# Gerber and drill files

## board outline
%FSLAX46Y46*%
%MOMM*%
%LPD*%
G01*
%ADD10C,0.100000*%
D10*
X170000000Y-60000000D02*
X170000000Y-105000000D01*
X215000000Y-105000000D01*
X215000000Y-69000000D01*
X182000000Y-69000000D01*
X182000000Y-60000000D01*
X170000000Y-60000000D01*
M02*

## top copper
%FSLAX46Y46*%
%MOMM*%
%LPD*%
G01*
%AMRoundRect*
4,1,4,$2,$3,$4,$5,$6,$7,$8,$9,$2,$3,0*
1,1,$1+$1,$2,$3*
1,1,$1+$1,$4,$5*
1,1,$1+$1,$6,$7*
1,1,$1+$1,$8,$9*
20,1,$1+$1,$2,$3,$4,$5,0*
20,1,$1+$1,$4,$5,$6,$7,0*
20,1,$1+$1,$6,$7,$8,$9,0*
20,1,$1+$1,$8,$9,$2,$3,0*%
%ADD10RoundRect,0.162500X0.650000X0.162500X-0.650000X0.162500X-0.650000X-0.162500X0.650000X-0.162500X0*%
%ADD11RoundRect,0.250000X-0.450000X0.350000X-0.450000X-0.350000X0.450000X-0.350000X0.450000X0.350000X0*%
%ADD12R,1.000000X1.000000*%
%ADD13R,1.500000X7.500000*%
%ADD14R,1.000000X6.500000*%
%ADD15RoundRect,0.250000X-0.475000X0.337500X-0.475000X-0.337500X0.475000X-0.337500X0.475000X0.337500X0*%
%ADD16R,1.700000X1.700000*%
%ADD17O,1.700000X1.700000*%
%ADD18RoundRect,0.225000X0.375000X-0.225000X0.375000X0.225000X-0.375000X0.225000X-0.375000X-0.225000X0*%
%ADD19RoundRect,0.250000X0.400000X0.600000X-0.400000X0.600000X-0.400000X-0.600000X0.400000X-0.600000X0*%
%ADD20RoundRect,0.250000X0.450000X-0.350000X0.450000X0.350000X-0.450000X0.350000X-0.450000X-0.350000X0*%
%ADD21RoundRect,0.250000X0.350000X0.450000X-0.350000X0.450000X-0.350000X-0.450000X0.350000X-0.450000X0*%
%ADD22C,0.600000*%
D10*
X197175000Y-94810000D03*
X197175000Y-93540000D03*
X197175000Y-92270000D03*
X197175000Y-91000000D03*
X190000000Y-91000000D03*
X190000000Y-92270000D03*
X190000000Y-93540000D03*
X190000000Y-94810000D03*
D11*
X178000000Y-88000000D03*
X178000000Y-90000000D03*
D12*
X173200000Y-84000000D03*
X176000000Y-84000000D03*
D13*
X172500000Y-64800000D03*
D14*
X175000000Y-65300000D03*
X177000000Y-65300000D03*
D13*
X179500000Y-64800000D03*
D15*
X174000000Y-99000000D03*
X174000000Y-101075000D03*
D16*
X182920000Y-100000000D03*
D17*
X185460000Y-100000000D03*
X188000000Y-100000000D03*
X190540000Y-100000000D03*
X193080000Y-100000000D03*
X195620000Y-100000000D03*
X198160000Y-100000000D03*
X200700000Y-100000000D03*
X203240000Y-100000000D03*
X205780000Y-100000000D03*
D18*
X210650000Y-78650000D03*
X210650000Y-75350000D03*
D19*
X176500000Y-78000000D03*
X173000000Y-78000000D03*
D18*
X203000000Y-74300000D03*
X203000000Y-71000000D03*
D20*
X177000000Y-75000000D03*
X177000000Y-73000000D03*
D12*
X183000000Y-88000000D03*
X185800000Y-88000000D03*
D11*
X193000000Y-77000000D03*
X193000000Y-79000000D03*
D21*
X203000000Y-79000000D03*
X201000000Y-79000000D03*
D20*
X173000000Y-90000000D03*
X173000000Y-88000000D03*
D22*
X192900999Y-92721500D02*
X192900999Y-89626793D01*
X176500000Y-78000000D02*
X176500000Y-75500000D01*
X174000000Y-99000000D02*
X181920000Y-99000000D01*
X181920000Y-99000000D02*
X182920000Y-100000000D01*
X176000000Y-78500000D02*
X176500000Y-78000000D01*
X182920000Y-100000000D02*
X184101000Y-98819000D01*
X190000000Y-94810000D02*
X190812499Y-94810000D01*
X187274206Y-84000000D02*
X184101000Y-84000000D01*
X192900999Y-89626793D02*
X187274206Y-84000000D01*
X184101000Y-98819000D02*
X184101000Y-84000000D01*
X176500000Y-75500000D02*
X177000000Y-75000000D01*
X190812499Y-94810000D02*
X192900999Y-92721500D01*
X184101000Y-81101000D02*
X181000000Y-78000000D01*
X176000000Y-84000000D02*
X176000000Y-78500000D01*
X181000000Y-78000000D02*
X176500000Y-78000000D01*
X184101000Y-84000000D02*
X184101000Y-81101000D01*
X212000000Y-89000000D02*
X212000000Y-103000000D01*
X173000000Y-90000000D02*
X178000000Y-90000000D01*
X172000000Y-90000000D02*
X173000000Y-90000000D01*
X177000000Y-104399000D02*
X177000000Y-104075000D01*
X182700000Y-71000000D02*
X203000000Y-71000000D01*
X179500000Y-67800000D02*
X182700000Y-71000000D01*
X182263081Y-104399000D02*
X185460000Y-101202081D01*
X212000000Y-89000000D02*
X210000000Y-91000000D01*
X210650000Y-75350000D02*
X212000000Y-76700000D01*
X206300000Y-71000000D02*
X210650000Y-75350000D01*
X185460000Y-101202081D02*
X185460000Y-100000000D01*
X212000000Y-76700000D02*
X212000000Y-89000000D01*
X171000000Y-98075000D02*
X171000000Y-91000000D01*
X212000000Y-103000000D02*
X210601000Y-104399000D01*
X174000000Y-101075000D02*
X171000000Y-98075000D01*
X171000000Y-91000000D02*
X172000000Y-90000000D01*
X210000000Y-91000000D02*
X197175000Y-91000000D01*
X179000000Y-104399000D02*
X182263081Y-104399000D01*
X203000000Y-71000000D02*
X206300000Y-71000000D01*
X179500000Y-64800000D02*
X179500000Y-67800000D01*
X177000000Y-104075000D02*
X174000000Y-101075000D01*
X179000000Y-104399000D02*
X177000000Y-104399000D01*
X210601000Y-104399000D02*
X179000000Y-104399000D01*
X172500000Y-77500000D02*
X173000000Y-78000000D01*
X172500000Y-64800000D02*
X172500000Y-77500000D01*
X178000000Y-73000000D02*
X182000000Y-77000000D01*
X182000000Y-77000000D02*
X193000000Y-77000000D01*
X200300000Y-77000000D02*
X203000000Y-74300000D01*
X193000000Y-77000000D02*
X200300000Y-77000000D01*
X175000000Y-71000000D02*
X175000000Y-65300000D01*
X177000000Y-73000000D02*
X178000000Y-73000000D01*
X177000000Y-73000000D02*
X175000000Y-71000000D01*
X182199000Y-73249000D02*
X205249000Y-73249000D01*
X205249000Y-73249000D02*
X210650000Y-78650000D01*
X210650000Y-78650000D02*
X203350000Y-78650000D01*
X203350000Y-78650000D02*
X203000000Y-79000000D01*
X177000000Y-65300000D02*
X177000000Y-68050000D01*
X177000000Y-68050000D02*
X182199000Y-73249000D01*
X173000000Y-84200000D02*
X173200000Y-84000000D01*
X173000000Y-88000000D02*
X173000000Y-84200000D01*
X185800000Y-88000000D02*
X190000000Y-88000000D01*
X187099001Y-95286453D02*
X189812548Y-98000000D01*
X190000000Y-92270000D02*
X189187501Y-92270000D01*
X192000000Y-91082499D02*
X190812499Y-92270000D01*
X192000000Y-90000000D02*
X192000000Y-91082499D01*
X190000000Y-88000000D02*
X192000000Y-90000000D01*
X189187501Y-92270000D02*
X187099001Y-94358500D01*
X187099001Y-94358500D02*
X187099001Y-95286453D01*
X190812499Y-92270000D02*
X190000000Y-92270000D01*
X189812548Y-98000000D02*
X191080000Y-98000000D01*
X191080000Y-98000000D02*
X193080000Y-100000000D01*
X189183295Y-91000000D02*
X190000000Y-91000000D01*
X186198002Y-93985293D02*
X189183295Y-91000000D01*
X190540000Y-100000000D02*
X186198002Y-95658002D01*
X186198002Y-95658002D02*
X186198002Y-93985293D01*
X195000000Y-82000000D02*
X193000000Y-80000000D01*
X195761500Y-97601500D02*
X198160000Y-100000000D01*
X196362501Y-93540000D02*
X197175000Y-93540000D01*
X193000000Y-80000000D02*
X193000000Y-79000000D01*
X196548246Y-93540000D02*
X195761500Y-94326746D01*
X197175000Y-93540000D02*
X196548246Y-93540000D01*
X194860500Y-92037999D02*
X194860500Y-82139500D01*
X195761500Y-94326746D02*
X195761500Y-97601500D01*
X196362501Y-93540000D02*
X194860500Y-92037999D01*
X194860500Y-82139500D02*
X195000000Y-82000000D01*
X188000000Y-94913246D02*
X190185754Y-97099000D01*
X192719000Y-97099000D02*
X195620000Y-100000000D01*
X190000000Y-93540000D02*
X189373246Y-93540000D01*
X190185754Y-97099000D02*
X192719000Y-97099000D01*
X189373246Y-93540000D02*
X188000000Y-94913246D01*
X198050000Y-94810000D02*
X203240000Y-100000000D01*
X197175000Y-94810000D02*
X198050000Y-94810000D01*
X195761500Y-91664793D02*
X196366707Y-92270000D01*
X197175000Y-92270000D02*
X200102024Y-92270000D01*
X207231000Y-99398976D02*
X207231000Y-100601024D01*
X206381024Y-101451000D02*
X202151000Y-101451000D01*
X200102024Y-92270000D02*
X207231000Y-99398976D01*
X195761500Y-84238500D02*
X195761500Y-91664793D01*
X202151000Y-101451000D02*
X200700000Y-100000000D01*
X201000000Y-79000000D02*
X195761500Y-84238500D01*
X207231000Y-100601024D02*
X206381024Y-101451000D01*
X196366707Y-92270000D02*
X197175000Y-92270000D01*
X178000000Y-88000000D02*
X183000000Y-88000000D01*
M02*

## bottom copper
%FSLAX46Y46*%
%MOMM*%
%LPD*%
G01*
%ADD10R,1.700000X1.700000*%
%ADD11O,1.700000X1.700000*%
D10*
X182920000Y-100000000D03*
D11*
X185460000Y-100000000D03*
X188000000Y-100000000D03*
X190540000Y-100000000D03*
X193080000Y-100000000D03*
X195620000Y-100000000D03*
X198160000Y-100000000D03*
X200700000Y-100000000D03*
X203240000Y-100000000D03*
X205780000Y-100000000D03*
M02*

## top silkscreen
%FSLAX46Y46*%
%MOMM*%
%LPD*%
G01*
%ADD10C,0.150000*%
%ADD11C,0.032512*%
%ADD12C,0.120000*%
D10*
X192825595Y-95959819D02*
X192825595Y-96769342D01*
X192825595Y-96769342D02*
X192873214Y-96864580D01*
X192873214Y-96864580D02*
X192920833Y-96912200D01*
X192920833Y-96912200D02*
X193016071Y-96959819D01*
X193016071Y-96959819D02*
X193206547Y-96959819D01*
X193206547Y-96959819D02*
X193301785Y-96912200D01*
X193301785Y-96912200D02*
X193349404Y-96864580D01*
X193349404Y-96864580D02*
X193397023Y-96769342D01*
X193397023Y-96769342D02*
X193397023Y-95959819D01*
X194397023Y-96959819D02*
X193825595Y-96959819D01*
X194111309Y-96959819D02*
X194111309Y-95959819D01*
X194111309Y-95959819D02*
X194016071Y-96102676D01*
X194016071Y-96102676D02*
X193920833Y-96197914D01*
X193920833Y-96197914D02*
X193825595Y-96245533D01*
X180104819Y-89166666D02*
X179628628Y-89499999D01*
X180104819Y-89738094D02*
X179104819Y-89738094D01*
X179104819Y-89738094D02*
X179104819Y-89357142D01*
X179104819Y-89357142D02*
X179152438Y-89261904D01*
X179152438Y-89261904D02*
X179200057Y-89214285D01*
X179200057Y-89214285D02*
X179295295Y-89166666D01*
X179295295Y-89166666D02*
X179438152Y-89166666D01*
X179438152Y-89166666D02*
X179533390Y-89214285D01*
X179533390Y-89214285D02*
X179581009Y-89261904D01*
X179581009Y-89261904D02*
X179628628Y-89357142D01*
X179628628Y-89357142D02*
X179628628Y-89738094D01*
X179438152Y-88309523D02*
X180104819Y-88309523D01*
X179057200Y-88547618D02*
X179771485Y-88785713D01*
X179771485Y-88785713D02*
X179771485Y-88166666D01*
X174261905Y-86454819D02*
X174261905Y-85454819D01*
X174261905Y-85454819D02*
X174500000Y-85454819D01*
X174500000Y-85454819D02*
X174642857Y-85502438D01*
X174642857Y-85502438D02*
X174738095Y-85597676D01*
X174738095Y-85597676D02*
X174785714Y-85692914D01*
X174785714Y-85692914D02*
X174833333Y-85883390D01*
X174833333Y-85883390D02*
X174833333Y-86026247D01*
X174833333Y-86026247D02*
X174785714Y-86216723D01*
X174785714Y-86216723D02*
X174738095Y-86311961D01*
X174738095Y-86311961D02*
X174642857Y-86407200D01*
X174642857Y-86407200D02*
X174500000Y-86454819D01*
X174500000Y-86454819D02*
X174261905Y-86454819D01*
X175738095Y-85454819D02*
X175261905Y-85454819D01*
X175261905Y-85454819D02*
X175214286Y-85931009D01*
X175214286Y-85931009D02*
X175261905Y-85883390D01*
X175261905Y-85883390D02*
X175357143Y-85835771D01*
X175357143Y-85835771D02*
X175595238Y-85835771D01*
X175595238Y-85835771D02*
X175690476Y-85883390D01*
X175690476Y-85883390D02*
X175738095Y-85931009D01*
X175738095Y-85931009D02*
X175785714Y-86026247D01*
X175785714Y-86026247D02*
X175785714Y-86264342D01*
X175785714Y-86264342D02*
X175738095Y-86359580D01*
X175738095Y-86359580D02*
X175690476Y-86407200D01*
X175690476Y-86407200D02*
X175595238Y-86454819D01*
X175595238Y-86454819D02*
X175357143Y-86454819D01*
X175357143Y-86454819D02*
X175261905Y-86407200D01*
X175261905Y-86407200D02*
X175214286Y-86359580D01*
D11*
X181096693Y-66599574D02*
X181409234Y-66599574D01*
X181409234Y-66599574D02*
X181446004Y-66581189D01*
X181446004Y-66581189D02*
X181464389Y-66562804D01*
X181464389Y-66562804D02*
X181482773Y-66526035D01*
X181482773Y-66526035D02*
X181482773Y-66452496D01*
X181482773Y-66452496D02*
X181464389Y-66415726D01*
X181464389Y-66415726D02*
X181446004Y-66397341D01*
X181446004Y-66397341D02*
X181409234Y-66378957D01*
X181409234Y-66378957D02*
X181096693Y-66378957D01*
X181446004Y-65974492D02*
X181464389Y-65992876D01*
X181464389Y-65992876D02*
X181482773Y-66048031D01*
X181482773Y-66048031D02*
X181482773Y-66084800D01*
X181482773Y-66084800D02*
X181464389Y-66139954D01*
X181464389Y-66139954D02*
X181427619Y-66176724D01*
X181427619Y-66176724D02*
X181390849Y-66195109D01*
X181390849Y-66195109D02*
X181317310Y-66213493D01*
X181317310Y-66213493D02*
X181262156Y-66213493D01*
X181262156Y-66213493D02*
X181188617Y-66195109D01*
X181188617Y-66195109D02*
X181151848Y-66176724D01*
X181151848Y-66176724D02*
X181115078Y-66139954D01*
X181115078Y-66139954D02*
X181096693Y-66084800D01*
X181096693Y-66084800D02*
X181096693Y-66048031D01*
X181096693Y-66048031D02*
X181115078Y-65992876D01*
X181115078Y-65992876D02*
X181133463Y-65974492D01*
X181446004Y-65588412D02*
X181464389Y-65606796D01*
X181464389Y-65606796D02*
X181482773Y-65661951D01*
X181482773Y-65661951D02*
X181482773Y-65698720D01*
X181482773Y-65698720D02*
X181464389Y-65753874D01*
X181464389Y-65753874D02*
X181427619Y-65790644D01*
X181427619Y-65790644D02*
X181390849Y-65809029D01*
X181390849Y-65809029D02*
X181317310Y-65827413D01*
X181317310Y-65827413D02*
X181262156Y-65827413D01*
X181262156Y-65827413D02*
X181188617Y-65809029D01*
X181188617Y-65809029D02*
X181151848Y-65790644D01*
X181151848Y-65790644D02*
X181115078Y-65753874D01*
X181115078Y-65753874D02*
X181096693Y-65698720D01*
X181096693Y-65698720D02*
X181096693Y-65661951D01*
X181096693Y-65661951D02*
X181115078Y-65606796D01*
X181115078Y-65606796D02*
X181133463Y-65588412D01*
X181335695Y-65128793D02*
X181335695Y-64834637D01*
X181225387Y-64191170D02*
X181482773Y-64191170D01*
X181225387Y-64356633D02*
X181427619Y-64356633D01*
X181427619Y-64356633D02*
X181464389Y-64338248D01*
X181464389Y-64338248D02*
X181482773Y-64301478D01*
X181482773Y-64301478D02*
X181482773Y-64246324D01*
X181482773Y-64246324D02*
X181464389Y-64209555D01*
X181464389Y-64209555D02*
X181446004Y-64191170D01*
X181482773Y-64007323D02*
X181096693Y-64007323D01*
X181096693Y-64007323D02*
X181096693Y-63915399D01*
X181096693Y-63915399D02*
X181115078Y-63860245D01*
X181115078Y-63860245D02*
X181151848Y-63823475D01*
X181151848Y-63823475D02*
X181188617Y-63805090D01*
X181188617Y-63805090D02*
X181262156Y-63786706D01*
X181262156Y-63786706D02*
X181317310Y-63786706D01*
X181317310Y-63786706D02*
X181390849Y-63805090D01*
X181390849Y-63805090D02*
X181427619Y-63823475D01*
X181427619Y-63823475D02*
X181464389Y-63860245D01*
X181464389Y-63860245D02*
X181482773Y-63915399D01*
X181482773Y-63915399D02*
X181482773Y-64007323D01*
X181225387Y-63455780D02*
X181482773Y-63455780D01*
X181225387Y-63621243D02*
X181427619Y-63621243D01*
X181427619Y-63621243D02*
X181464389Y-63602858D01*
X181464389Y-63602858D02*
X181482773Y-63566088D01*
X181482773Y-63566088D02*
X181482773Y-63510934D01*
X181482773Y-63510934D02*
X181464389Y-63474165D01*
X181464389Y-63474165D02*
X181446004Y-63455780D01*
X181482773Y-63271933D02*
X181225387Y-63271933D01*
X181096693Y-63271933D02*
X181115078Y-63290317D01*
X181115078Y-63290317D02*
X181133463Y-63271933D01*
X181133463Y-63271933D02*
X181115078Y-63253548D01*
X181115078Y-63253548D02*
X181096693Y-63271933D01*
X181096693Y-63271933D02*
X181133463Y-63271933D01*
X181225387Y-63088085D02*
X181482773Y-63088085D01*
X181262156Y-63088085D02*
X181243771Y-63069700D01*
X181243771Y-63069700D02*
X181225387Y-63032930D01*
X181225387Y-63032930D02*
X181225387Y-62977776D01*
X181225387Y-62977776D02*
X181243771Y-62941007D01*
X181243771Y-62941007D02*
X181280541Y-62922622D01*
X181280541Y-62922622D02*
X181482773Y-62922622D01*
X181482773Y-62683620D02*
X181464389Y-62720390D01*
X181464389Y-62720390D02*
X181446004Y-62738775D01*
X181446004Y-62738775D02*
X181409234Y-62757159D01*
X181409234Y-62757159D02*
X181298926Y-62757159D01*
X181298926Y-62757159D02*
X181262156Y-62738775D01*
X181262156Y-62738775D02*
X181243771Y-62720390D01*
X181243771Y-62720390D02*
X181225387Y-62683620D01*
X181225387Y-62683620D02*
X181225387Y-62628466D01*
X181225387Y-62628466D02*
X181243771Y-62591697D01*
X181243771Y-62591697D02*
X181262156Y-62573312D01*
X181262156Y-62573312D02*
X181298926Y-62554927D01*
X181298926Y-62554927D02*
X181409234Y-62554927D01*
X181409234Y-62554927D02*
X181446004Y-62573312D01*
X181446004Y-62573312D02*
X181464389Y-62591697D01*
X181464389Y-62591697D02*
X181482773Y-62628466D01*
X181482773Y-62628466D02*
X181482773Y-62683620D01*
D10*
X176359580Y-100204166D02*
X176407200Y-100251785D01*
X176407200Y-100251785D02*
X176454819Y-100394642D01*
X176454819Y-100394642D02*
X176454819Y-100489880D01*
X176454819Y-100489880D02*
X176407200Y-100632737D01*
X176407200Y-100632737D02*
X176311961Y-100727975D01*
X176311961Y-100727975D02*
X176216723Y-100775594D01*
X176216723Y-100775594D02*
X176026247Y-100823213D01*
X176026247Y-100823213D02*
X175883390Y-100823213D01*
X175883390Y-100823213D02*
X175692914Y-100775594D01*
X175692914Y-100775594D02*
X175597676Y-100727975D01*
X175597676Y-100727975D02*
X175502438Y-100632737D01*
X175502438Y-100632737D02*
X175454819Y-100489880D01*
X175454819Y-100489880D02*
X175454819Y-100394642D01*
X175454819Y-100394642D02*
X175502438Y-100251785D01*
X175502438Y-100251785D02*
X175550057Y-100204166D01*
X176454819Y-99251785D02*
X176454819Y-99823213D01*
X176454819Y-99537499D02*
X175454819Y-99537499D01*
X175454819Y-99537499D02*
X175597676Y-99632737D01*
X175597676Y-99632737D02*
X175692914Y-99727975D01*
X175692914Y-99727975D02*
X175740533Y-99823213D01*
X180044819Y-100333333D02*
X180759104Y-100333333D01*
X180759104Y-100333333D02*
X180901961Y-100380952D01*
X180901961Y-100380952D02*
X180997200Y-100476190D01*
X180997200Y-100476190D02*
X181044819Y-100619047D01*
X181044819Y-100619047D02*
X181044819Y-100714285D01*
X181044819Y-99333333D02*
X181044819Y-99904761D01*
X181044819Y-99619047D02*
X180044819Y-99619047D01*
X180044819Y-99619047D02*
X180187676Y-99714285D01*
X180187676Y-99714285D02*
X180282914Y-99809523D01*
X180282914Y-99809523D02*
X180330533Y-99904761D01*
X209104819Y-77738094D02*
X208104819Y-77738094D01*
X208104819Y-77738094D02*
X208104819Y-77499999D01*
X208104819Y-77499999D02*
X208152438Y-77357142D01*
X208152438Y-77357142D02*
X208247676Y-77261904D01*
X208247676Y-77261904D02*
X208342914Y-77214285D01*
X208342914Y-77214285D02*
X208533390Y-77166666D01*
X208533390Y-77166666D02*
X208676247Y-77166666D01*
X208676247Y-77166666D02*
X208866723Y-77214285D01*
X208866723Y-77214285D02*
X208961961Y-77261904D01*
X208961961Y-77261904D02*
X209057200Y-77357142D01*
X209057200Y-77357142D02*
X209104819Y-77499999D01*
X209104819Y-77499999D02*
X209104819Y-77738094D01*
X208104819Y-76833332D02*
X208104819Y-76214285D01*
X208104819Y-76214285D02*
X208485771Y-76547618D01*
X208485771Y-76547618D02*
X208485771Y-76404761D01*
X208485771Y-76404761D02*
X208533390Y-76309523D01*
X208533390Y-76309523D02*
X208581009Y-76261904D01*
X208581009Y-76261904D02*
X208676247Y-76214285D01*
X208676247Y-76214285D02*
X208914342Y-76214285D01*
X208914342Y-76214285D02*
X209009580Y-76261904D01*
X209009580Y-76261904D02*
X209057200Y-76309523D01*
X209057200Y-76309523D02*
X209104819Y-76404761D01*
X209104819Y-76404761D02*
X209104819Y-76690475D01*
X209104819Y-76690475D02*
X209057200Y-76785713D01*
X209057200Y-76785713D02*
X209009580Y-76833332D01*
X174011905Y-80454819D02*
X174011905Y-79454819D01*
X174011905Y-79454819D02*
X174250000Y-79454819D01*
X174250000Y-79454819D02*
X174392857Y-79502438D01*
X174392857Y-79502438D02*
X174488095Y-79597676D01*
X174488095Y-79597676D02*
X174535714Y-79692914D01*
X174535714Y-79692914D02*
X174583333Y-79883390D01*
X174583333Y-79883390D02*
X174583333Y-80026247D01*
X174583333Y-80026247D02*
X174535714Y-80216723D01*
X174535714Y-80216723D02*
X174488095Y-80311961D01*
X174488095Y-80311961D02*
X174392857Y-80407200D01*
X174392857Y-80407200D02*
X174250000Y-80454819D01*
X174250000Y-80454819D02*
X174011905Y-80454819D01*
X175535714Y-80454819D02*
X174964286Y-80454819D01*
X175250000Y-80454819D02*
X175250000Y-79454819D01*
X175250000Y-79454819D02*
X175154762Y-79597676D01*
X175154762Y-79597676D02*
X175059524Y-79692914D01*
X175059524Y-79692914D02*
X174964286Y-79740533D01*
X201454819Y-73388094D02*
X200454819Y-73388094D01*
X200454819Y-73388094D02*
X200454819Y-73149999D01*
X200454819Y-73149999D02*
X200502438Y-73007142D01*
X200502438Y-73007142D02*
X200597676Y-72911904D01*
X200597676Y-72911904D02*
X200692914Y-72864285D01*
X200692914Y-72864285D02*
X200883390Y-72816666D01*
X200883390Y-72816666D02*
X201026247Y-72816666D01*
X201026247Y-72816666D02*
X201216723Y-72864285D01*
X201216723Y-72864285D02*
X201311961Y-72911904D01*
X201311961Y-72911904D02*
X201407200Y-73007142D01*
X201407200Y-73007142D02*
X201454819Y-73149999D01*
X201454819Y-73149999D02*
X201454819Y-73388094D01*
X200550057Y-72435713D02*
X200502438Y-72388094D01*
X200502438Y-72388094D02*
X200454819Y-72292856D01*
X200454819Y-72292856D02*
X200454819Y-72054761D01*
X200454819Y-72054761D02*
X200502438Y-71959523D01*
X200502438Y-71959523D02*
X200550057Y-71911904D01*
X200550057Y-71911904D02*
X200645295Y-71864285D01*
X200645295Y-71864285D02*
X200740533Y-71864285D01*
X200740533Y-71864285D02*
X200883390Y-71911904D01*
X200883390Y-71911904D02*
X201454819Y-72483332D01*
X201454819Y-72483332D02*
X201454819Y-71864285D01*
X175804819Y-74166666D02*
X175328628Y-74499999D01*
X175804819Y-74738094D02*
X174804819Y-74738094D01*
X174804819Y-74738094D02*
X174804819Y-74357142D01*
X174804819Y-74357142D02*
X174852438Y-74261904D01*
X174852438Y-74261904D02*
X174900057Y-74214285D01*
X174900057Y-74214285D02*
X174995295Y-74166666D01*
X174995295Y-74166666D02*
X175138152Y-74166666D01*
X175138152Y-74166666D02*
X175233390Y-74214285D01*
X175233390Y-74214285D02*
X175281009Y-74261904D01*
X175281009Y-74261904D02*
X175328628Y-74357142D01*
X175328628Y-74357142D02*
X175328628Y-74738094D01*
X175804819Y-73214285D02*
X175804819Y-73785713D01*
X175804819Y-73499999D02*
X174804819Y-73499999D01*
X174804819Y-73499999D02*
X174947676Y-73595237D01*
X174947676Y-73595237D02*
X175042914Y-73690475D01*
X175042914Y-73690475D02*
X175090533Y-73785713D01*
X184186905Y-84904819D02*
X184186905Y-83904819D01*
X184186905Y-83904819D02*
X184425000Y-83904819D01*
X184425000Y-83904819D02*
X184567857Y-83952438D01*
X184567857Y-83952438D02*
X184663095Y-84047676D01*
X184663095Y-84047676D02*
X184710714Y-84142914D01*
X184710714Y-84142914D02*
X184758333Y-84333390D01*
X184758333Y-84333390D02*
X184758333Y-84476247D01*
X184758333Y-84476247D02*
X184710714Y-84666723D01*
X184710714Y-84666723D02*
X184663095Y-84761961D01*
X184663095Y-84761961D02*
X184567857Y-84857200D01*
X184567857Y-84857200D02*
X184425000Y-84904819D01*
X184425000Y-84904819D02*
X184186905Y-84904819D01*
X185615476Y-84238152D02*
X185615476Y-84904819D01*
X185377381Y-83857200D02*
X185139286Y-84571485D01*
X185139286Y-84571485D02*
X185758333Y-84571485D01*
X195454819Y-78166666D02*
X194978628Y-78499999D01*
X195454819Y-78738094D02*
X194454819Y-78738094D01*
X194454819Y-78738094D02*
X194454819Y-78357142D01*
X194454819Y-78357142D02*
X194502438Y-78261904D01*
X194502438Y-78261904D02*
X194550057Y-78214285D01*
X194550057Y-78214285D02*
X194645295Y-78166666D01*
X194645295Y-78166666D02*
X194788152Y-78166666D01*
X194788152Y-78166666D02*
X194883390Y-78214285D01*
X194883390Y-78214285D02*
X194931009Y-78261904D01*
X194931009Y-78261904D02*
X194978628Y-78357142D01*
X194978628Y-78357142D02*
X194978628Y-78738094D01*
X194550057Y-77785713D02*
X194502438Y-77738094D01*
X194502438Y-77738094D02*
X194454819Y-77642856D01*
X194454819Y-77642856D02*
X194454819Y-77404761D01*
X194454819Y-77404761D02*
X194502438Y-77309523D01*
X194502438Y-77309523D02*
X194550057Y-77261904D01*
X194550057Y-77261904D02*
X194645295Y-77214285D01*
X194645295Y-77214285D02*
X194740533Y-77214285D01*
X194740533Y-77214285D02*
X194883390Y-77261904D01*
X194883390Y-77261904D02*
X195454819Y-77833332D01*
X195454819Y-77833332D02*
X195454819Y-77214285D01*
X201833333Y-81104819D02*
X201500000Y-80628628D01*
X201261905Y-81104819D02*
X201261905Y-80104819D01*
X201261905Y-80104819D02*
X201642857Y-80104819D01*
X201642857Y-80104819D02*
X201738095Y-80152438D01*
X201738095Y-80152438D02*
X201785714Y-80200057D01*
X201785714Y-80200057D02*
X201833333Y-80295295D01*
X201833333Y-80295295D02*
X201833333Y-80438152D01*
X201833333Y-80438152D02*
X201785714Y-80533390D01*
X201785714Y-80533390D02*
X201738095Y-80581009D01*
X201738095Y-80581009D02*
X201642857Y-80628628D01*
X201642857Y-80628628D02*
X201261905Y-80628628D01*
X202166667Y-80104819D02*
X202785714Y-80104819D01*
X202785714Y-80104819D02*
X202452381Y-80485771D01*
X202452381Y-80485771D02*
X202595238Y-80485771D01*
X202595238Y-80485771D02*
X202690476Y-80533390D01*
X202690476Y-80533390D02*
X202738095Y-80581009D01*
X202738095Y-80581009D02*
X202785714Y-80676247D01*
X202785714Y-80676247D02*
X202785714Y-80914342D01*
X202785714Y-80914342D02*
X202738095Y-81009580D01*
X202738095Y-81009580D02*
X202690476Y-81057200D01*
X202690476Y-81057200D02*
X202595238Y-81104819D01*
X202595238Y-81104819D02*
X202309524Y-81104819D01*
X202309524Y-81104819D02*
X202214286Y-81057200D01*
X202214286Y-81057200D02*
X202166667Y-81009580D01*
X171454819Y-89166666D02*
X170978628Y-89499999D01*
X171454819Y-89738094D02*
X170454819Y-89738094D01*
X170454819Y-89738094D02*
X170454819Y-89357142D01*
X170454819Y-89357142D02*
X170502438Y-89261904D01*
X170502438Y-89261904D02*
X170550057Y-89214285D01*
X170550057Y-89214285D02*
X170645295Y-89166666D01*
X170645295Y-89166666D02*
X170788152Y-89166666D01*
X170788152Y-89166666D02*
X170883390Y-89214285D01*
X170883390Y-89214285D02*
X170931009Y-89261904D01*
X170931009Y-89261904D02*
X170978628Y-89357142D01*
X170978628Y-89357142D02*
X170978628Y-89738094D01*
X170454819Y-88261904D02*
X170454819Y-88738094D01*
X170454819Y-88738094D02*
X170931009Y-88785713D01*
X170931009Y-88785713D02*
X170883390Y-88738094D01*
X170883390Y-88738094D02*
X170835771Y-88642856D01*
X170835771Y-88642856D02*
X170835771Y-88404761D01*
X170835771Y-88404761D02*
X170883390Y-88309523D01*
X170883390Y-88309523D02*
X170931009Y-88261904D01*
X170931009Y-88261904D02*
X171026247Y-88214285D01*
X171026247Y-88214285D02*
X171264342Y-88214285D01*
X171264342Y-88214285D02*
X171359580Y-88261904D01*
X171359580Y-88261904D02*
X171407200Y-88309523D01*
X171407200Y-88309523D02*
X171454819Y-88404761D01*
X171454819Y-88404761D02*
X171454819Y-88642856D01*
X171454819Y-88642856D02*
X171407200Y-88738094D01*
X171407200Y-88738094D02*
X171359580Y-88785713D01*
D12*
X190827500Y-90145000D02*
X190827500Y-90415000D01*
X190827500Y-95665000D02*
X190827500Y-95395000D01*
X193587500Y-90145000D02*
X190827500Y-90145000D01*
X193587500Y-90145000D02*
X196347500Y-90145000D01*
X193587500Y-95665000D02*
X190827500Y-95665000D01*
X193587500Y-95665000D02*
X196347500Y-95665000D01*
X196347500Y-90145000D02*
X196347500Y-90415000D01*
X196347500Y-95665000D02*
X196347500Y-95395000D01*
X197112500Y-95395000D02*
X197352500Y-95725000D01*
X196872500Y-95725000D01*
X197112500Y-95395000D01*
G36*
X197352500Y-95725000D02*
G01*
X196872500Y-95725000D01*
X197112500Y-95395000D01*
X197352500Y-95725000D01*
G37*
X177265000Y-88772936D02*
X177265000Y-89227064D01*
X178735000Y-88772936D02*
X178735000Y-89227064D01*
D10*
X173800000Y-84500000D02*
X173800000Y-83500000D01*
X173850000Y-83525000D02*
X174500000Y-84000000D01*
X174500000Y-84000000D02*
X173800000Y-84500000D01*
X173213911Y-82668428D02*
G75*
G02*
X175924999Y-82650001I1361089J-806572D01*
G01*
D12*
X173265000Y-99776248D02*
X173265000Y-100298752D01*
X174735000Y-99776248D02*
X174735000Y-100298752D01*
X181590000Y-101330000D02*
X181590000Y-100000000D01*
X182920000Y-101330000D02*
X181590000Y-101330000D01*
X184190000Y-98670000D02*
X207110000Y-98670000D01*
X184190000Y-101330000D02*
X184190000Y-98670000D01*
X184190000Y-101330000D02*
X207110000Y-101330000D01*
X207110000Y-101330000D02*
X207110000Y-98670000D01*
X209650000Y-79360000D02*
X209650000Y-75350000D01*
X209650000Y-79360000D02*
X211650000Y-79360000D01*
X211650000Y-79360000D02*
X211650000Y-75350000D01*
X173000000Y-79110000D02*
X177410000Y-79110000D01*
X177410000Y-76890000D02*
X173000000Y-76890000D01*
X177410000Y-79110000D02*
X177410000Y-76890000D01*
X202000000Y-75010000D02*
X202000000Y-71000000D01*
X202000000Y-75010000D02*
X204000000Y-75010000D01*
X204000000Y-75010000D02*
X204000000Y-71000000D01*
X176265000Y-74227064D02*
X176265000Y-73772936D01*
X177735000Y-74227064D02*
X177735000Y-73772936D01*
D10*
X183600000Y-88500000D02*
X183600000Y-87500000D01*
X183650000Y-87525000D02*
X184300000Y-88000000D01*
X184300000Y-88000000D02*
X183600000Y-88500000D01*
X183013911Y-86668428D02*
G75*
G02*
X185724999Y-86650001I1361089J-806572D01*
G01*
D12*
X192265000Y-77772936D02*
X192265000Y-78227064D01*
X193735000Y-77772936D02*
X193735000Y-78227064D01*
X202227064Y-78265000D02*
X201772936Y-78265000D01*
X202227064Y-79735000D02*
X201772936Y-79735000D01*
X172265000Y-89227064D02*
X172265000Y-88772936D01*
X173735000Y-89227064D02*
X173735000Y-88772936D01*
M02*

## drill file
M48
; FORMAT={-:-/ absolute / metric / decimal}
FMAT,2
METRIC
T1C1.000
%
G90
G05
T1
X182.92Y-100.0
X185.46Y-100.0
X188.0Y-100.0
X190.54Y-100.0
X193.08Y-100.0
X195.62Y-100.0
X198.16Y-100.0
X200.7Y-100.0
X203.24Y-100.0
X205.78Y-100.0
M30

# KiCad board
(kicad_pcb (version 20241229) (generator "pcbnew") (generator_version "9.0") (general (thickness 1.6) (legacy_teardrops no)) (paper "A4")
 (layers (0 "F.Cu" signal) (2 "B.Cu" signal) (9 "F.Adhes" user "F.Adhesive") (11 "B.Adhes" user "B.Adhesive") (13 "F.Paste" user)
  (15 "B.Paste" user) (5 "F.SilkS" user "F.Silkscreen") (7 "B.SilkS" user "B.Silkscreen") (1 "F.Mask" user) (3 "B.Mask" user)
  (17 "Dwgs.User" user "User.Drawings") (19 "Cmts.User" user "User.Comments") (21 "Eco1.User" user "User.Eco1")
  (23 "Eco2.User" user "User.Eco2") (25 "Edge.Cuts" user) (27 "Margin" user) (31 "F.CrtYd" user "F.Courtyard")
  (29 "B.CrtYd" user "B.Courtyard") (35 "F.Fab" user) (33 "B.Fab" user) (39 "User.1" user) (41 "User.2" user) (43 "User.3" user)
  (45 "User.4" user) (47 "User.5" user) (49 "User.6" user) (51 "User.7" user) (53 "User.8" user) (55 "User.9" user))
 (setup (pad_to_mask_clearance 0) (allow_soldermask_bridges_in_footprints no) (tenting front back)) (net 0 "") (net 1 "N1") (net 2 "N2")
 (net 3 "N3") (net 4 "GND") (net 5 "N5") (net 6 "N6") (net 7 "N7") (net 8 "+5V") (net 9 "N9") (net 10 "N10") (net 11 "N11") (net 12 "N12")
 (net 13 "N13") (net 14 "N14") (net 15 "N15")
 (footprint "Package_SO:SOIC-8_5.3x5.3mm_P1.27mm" (layer "F.Cu") (at 193.5875 92.905 180)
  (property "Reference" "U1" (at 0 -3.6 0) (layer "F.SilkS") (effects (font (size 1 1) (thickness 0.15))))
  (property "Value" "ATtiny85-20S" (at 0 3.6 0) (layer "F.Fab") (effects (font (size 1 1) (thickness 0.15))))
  (fp_line (start 2.76 2.76) (end 2.76 2.49) (stroke (width 0.12) (type solid)) (layer "F.SilkS"))
  (fp_line (start 2.76 -2.76) (end 2.76 -2.49) (stroke (width 0.12) (type solid)) (layer "F.SilkS"))
  (fp_line (start 0 2.76) (end 2.76 2.76) (stroke (width 0.12) (type solid)) (layer "F.SilkS"))
  (fp_line (start 0 2.76) (end -2.76 2.76) (stroke (width 0.12) (type solid)) (layer "F.SilkS"))
  (fp_line (start 0 -2.76) (end 2.76 -2.76) (stroke (width 0.12) (type solid)) (layer "F.SilkS"))
  (fp_line (start 0 -2.76) (end -2.76 -2.76) (stroke (width 0.12) (type solid)) (layer "F.SilkS"))
  (fp_line (start -2.76 2.76) (end -2.76 2.49) (stroke (width 0.12) (type solid)) (layer "F.SilkS"))
  (fp_line (start -2.76 -2.76) (end -2.76 -2.49) (stroke (width 0.12) (type solid)) (layer "F.SilkS"))
  (fp_poly (pts (xy -3.525 -2.49) (xy -3.765 -2.82) (xy -3.285 -2.82)) (stroke (width 0.12) (type solid)) (fill yes) (layer "F.SilkS"))
  (pad "1" smd roundrect (at -3.5875 -1.905 180) (size 1.625 0.65) (layers "F.Cu" "F.Mask" "F.Paste") (roundrect_rratio 0.25) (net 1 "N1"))
  (pad "2" smd roundrect (at -3.5875 -0.635 180) (size 1.625 0.65) (layers "F.Cu" "F.Mask" "F.Paste") (roundrect_rratio 0.25) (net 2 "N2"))
  (pad "3" smd roundrect (at -3.5875 0.635 180) (size 1.625 0.65) (layers "F.Cu" "F.Mask" "F.Paste") (roundrect_rratio 0.25) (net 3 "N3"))
  (pad "4" smd roundrect (at -3.5875 1.905 180) (size 1.625 0.65) (layers "F.Cu" "F.Mask" "F.Paste") (roundrect_rratio 0.25) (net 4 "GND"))
  (pad "5" smd roundrect (at 3.5875 1.905 180) (size 1.625 0.65) (layers "F.Cu" "F.Mask" "F.Paste") (roundrect_rratio 0.25) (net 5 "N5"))
  (pad "6" smd roundrect (at 3.5875 0.635 180) (size 1.625 0.65) (layers "F.Cu" "F.Mask" "F.Paste") (roundrect_rratio 0.25) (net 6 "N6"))
  (pad "7" smd roundrect (at 3.5875 -0.635 180) (size 1.625 0.65) (layers "F.Cu" "F.Mask" "F.Paste") (roundrect_rratio 0.25) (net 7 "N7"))
  (pad "8" smd roundrect (at 3.5875 -1.905 180) (size 1.625 0.65) (layers "F.Cu" "F.Mask" "F.Paste") (roundrect_rratio 0.25) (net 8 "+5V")))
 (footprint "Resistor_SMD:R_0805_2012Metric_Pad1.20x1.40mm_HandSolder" (layer "F.Cu") (at 178 89 -90)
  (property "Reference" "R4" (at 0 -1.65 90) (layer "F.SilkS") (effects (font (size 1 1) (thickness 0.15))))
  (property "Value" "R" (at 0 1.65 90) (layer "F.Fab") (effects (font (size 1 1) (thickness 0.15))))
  (fp_line (start -0.227064 0.735) (end 0.227064 0.735) (stroke (width 0.12) (type solid)) (layer "F.SilkS"))
  (fp_line (start -0.227064 -0.735) (end 0.227064 -0.735) (stroke (width 0.12) (type solid)) (layer "F.SilkS"))
  (pad "1" smd roundrect (at -1 0 270) (size 1.2 1.4) (layers "F.Cu" "F.Mask" "F.Paste") (roundrect_rratio 0.208333) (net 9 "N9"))
  (pad "2" smd roundrect (at 1 0 270) (size 1.2 1.4) (layers "F.Cu" "F.Mask" "F.Paste") (roundrect_rratio 0.208333) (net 4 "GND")))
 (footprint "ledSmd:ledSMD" (layer "F.Cu") (at 175 84)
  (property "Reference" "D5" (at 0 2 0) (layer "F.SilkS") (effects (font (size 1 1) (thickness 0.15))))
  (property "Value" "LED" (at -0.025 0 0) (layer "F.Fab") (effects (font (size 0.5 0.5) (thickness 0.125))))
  (fp_line (start -1.2 0.5) (end -1.2 -0.5) (stroke (width 0.15) (type solid)) (layer "F.SilkS"))
  (fp_line (start -1.15 -0.475) (end -0.5 0) (stroke (width 0.15) (type solid)) (layer "F.SilkS"))
  (fp_line (start -0.5 0) (end -1.2 0.5) (stroke (width 0.15) (type solid)) (layer "F.SilkS"))
  (fp_arc (start -1.786089 -1.331572) (mid -0.435753 -2.107089) (end 0.924999 -1.349999) (stroke (width 0.15) (type solid))
   (layer "F.SilkS"))
  (pad "1" smd rect (at -1.8 0) (size 1 1) (layers "F.Cu" "F.Mask" "F.Paste") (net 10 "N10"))
  (pad "2" smd rect (at 1 0) (size 1 1) (layers "F.Cu" "F.Mask" "F.Paste") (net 8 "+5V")))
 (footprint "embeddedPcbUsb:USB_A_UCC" (layer "F.Cu") (at 176 65 -90)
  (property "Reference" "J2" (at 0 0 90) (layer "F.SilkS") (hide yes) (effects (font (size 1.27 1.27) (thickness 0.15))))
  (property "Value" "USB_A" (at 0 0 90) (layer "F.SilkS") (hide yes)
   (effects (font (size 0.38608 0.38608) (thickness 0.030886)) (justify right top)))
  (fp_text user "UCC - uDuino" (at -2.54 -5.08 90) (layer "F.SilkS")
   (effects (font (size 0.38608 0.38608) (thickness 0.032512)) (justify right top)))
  (pad "1" smd rect (at -0.2 3.5 270) (size 7.5 1.5) (layers "F.Cu" "F.Mask" "F.Paste") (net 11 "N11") (solder_mask_margin 0.1016))
  (pad "2" smd rect (at 0.3 1 270) (size 6.5 1) (layers "F.Cu" "F.Mask" "F.Paste") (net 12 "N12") (solder_mask_margin 0.1016))
  (pad "3" smd rect (at 0.3 -1 270) (size 6.5 1) (layers "F.Cu" "F.Mask" "F.Paste") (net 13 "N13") (solder_mask_margin 0.1016))
  (pad "4" smd rect (at -0.2 -3.5 270) (size 7.5 1.5) (layers "F.Cu" "F.Mask" "F.Paste") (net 4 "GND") (solder_mask_margin 0.1016)))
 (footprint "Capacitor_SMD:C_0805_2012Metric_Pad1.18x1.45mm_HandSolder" (layer "F.Cu") (at 174 100.0375 -90)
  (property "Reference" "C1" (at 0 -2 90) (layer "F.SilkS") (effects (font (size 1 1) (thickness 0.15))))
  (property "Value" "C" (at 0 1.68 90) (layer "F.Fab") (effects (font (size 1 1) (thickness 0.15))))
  (fp_line (start -0.261252 0.735) (end 0.261252 0.735) (stroke (width 0.12) (type solid)) (layer "F.SilkS"))
  (fp_line (start -0.261252 -0.735) (end 0.261252 -0.735) (stroke (width 0.12) (type solid)) (layer "F.SilkS"))
  (pad "1" smd roundrect (at -1.0375 0 270) (size 1.175 1.45) (layers "F.Cu" "F.Mask" "F.Paste") (roundrect_rratio 0.212766) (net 8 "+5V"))
  (pad "2" smd roundrect (at 1.0375 0 270) (size 1.175 1.45) (layers "F.Cu" "F.Mask" "F.Paste") (roundrect_rratio 0.212766) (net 4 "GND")))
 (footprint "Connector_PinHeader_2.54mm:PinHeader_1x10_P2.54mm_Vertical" (layer "F.Cu") (at 182.92 100 90)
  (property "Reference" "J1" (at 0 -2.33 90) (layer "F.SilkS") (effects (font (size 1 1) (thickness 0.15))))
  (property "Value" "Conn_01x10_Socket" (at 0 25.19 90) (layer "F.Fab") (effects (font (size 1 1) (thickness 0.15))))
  (fp_line (start -1.33 -1.33) (end 0 -1.33) (stroke (width 0.12) (type solid)) (layer "F.SilkS"))
  (fp_line (start -1.33 0) (end -1.33 -1.33) (stroke (width 0.12) (type solid)) (layer "F.SilkS"))
  (fp_line (start 1.33 1.27) (end 1.33 24.19) (stroke (width 0.12) (type solid)) (layer "F.SilkS"))
  (fp_line (start -1.33 1.27) (end 1.33 1.27) (stroke (width 0.12) (type solid)) (layer "F.SilkS"))
  (fp_line (start -1.33 1.27) (end -1.33 24.19) (stroke (width 0.12) (type solid)) (layer "F.SilkS"))
  (fp_line (start -1.33 24.19) (end 1.33 24.19) (stroke (width 0.12) (type solid)) (layer "F.SilkS"))
  (pad "1" thru_hole rect (at 0 0 90) (size 1.7 1.7) (drill 1) (layers "*.Cu" "*.Mask") (remove_unused_layers no) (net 8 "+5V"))
  (pad "2" thru_hole oval (at 0 2.54 90) (size 1.7 1.7) (drill 1) (layers "*.Cu" "*.Mask") (remove_unused_layers no) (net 4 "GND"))
  (pad "3" thru_hole oval (at 0 5.08 90) (size 1.7 1.7) (drill 1) (layers "*.Cu" "*.Mask") (remove_unused_layers no) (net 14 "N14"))
  (pad "4" thru_hole oval (at 0 7.62 90) (size 1.7 1.7) (drill 1) (layers "*.Cu" "*.Mask") (remove_unused_layers no) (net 5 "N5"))
  (pad "5" thru_hole oval (at 0 10.16 90) (size 1.7 1.7) (drill 1) (layers "*.Cu" "*.Mask") (remove_unused_layers no) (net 6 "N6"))
  (pad "6" thru_hole oval (at 0 12.7 90) (size 1.7 1.7) (drill 1) (layers "*.Cu" "*.Mask") (remove_unused_layers no) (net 7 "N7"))
  (pad "7" thru_hole oval (at 0 15.24 90) (size 1.7 1.7) (drill 1) (layers "*.Cu" "*.Mask") (remove_unused_layers no) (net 2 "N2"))
  (pad "8" thru_hole oval (at 0 17.78 90) (size 1.7 1.7) (drill 1) (layers "*.Cu" "*.Mask") (remove_unused_layers no) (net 3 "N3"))
  (pad "9" thru_hole oval (at 0 20.32 90) (size 1.7 1.7) (drill 1) (layers "*.Cu" "*.Mask") (remove_unused_layers no) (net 1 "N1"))
  (pad "10" thru_hole oval (at 0 22.86 90) (size 1.7 1.7) (drill 1) (layers "*.Cu" "*.Mask") (remove_unused_layers no) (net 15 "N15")))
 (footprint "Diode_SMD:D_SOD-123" (layer "F.Cu") (at 210.65 77 90)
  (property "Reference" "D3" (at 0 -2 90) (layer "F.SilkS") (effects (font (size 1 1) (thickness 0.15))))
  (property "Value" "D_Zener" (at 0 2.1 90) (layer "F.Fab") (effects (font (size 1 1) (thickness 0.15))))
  (fp_line (start -2.36 -1) (end 1.65 -1) (stroke (width 0.12) (type solid)) (layer "F.SilkS"))
  (fp_line (start -2.36 -1) (end -2.36 1) (stroke (width 0.12) (type solid)) (layer "F.SilkS"))
  (fp_line (start -2.36 1) (end 1.65 1) (stroke (width 0.12) (type solid)) (layer "F.SilkS"))
  (pad "1" smd roundrect (at -1.65 0 90) (size 0.9 1.2) (layers "F.Cu" "F.Mask" "F.Paste") (roundrect_rratio 0.25) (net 13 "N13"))
  (pad "2" smd roundrect (at 1.65 0 90) (size 0.9 1.2) (layers "F.Cu" "F.Mask" "F.Paste") (roundrect_rratio 0.25) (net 4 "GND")))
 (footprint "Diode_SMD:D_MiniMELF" (layer "F.Cu") (at 174.75 78 180)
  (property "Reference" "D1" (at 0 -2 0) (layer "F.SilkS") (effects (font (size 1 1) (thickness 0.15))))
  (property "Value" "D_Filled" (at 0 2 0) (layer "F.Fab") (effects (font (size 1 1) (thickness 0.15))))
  (fp_line (start 1.75 -1.11) (end -2.66 -1.11) (stroke (width 0.12) (type solid)) (layer "F.SilkS"))
  (fp_line (start -2.66 1.11) (end 1.75 1.11) (stroke (width 0.12) (type solid)) (layer "F.SilkS"))
  (fp_line (start -2.66 -1.11) (end -2.66 1.11) (stroke (width 0.12) (type solid)) (layer "F.SilkS"))
  (pad "1" smd roundrect (at -1.75 0 180) (size 1.3 1.7) (layers "F.Cu" "F.Mask" "F.Paste") (roundrect_rratio 0.1923076923) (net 8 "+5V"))
  (pad "2" smd roundrect (at 1.75 0 180) (size 1.3 1.7) (layers "F.Cu" "F.Mask" "F.Paste") (roundrect_rratio 0.1923076923) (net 11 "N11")))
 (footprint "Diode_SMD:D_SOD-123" (layer "F.Cu") (at 203 72.65 90)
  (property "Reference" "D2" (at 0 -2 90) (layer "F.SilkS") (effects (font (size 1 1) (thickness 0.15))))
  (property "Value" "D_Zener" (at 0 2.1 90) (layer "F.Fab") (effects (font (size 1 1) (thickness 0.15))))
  (fp_line (start -2.36 -1) (end 1.65 -1) (stroke (width 0.12) (type solid)) (layer "F.SilkS"))
  (fp_line (start -2.36 -1) (end -2.36 1) (stroke (width 0.12) (type solid)) (layer "F.SilkS"))
  (fp_line (start -2.36 1) (end 1.65 1) (stroke (width 0.12) (type solid)) (layer "F.SilkS"))
  (pad "1" smd roundrect (at -1.65 0 90) (size 0.9 1.2) (layers "F.Cu" "F.Mask" "F.Paste") (roundrect_rratio 0.25) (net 12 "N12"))
  (pad "2" smd roundrect (at 1.65 0 90) (size 0.9 1.2) (layers "F.Cu" "F.Mask" "F.Paste") (roundrect_rratio 0.25) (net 4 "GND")))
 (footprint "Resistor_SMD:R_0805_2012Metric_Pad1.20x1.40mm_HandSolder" (layer "F.Cu") (at 177 74 90)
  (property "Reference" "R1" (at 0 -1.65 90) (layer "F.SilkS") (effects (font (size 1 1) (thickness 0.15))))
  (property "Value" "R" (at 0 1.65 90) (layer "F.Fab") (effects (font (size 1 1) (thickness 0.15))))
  (fp_line (start -0.227064 -0.735) (end 0.227064 -0.735) (stroke (width 0.12) (type solid)) (layer "F.SilkS"))
  (fp_line (start -0.227064 0.735) (end 0.227064 0.735) (stroke (width 0.12) (type solid)) (layer "F.SilkS"))
  (pad "1" smd roundrect (at -1 0 90) (size 1.2 1.4) (layers "F.Cu" "F.Mask" "F.Paste") (roundrect_rratio 0.208333) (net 8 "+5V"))
  (pad "2" smd roundrect (at 1 0 90) (size 1.2 1.4) (layers "F.Cu" "F.Mask" "F.Paste") (roundrect_rratio 0.208333) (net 12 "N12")))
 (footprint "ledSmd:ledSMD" (layer "F.Cu") (at 184.8 88)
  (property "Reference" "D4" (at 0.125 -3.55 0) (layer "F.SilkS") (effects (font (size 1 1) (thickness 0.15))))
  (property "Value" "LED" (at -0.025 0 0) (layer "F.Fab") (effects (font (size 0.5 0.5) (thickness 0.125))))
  (fp_line (start -1.2 0.5) (end -1.2 -0.5) (stroke (width 0.15) (type solid)) (layer "F.SilkS"))
  (fp_line (start -1.15 -0.475) (end -0.5 0) (stroke (width 0.15) (type solid)) (layer "F.SilkS"))
  (fp_line (start -0.5 0) (end -1.2 0.5) (stroke (width 0.15) (type solid)) (layer "F.SilkS"))
  (fp_arc (start -1.786089 -1.331572) (mid -0.435753 -2.107089) (end 0.924999 -1.349999) (stroke (width 0.15) (type solid))
   (layer "F.SilkS"))
  (pad "1" smd rect (at -1.8 0) (size 1 1) (layers "F.Cu" "F.Mask" "F.Paste") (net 9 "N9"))
  (pad "2" smd rect (at 1 0) (size 1 1) (layers "F.Cu" "F.Mask" "F.Paste") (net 6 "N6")))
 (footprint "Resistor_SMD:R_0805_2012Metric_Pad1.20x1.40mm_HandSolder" (layer "F.Cu") (at 193 78 -90)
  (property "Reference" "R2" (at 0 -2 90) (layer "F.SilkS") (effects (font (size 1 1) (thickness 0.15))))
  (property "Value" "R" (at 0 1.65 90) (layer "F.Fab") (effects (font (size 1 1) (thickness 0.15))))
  (fp_line (start -0.227064 0.735) (end 0.227064 0.735) (stroke (width 0.12) (type solid)) (layer "F.SilkS"))
  (fp_line (start -0.227064 -0.735) (end 0.227064 -0.735) (stroke (width 0.12) (type solid)) (layer "F.SilkS"))
  (pad "1" smd roundrect (at -1 0 270) (size 1.2 1.4) (layers "F.Cu" "F.Mask" "F.Paste") (roundrect_rratio 0.208333) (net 12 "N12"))
  (pad "2" smd roundrect (at 1 0 270) (size 1.2 1.4) (layers "F.Cu" "F.Mask" "F.Paste") (roundrect_rratio 0.208333) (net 2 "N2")))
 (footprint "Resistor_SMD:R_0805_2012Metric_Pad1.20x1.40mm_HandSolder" (layer "F.Cu") (at 202 79 180)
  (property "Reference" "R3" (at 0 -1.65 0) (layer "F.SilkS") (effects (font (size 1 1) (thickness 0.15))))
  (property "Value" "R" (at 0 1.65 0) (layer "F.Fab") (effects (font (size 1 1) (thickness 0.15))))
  (fp_line (start -0.227064 0.735) (end 0.227064 0.735) (stroke (width 0.12) (type solid)) (layer "F.SilkS"))
  (fp_line (start -0.227064 -0.735) (end 0.227064 -0.735) (stroke (width 0.12) (type solid)) (layer "F.SilkS"))
  (pad "1" smd roundrect (at -1 0 180) (size 1.2 1.4) (layers "F.Cu" "F.Mask" "F.Paste") (roundrect_rratio 0.208333) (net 13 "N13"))
  (pad "2" smd roundrect (at 1 0 180) (size 1.2 1.4) (layers "F.Cu" "F.Mask" "F.Paste") (roundrect_rratio 0.208333) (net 3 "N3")))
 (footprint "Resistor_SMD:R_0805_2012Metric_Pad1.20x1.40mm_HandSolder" (layer "F.Cu") (at 173 89 90)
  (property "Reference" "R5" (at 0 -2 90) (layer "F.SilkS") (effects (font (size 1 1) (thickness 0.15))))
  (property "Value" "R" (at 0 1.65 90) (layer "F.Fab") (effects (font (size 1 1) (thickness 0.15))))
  (fp_line (start -0.227064 -0.735) (end 0.227064 -0.735) (stroke (width 0.12) (type solid)) (layer "F.SilkS"))
  (fp_line (start -0.227064 0.735) (end 0.227064 0.735) (stroke (width 0.12) (type solid)) (layer "F.SilkS"))
  (pad "1" smd roundrect (at -1 0 90) (size 1.2 1.4) (layers "F.Cu" "F.Mask" "F.Paste") (roundrect_rratio 0.208333) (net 4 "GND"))
  (pad "2" smd roundrect (at 1 0 90) (size 1.2 1.4) (layers "F.Cu" "F.Mask" "F.Paste") (roundrect_rratio 0.208333) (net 10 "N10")))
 (gr_poly
  (pts (xy 170 60) (xy 170 105) (xy 215 105) (xy 215 69) (xy 182 69) (xy 182 60)) (stroke (width 0.1) (type solid)) (fill no)
  (layer "Edge.Cuts"))
 (segment (start 192.900999 92.7215) (end 192.900999 89.626793) (width 0.6) (layer "F.Cu") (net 8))
 (segment (start 176.5 78) (end 176.5 75.5) (width 0.6) (layer "F.Cu") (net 8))
 (segment (start 174 99) (end 181.92 99) (width 0.6) (layer "F.Cu") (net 8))
 (segment (start 181.92 99) (end 182.92 100) (width 0.6) (layer "F.Cu") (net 8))
 (segment (start 176 78.5) (end 176.5 78) (width 0.6) (layer "F.Cu") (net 8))
 (segment (start 182.92 100) (end 184.101 98.819) (width 0.6) (layer "F.Cu") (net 8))
 (segment (start 190 94.81) (end 190.812499 94.81) (width 0.6) (layer "F.Cu") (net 8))
 (segment (start 187.274206 84) (end 184.101 84) (width 0.6) (layer "F.Cu") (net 8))
 (segment (start 192.900999 89.626793) (end 187.274206 84) (width 0.6) (layer "F.Cu") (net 8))
 (segment (start 184.101 98.819) (end 184.101 84) (width 0.6) (layer "F.Cu") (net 8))
 (segment (start 176.5 75.5) (end 177 75) (width 0.6) (layer "F.Cu") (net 8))
 (segment (start 190.812499 94.81) (end 192.900999 92.7215) (width 0.6) (layer "F.Cu") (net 8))
 (segment (start 184.101 81.101) (end 181 78) (width 0.6) (layer "F.Cu") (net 8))
 (segment (start 176 84) (end 176 78.5) (width 0.6) (layer "F.Cu") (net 8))
 (segment (start 181 78) (end 176.5 78) (width 0.6) (layer "F.Cu") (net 8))
 (segment (start 184.101 84) (end 184.101 81.101) (width 0.6) (layer "F.Cu") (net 8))
 (segment (start 212 89) (end 212 103) (width 0.6) (layer "F.Cu") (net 4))
 (segment (start 173 90) (end 178 90) (width 0.6) (layer "F.Cu") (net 4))
 (segment (start 172 90) (end 173 90) (width 0.6) (layer "F.Cu") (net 4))
 (segment (start 177 104.399) (end 177 104.075) (width 0.6) (layer "F.Cu") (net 4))
 (segment (start 182.7 71) (end 203 71) (width 0.6) (layer "F.Cu") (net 4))
 (segment (start 179.5 67.8) (end 182.7 71) (width 0.6) (layer "F.Cu") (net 4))
 (segment (start 182.263081 104.399) (end 185.46 101.202081) (width 0.6) (layer "F.Cu") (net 4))
 (segment (start 212 89) (end 210 91) (width 0.6) (layer "F.Cu") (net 4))
 (segment (start 210.65 75.35) (end 212 76.7) (width 0.6) (layer "F.Cu") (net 4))
 (segment (start 206.3 71) (end 210.65 75.35) (width 0.6) (layer "F.Cu") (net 4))
 (segment (start 185.46 101.202081) (end 185.46 100) (width 0.6) (layer "F.Cu") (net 4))
 (segment (start 212 76.7) (end 212 89) (width 0.6) (layer "F.Cu") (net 4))
 (segment (start 171 98.075) (end 171 91) (width 0.6) (layer "F.Cu") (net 4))
 (segment (start 212 103) (end 210.601 104.399) (width 0.6) (layer "F.Cu") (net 4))
 (segment (start 174 101.075) (end 171 98.075) (width 0.6) (layer "F.Cu") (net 4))
 (segment (start 171 91) (end 172 90) (width 0.6) (layer "F.Cu") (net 4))
 (segment (start 210 91) (end 197.175 91) (width 0.6) (layer "F.Cu") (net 4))
 (segment (start 179 104.399) (end 182.263081 104.399) (width 0.6) (layer "F.Cu") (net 4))
 (segment (start 203 71) (end 206.3 71) (width 0.6) (layer "F.Cu") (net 4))
 (segment (start 179.5 64.8) (end 179.5 67.8) (width 0.6) (layer "F.Cu") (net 4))
 (segment (start 177 104.075) (end 174 101.075) (width 0.6) (layer "F.Cu") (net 4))
 (segment (start 179 104.399) (end 177 104.399) (width 0.6) (layer "F.Cu") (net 4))
 (segment (start 210.601 104.399) (end 179 104.399) (width 0.6) (layer "F.Cu") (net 4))
 (segment (start 172.5 77.5) (end 173 78) (width 0.6) (layer "F.Cu") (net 11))
 (segment (start 172.5 64.8) (end 172.5 77.5) (width 0.6) (layer "F.Cu") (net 11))
 (segment (start 178 73) (end 182 77) (width 0.6) (layer "F.Cu") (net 12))
 (segment (start 182 77) (end 193 77) (width 0.6) (layer "F.Cu") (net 12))
 (segment (start 200.3 77) (end 203 74.3) (width 0.6) (layer "F.Cu") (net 12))
 (segment (start 193 77) (end 200.3 77) (width 0.6) (layer "F.Cu") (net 12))
 (segment (start 175 71) (end 175 65.3) (width 0.6) (layer "F.Cu") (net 12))
 (segment (start 177 73) (end 178 73) (width 0.6) (layer "F.Cu") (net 12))
 (segment (start 177 73) (end 175 71) (width 0.6) (layer "F.Cu") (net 12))
 (segment (start 182.199 73.249) (end 205.249 73.249) (width 0.6) (layer "F.Cu") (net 13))
 (segment (start 205.249 73.249) (end 210.65 78.65) (width 0.6) (layer "F.Cu") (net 13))
 (segment (start 210.65 78.65) (end 203.35 78.65) (width 0.6) (layer "F.Cu") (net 13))
 (segment (start 203.35 78.65) (end 203 79) (width 0.6) (layer "F.Cu") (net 13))
 (segment (start 177 65.3) (end 177 68.05) (width 0.6) (layer "F.Cu") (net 13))
 (segment (start 177 68.05) (end 182.199 73.249) (width 0.6) (layer "F.Cu") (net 13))
 (segment (start 173 84.2) (end 173.2 84) (width 0.6) (layer "F.Cu") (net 10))
 (segment (start 173 88) (end 173 84.2) (width 0.6) (layer "F.Cu") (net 10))
 (segment (start 185.8 88) (end 190 88) (width 0.6) (layer "F.Cu") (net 6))
 (segment (start 187.099001 95.286453) (end 189.812548 98) (width 0.6) (layer "F.Cu") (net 6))
 (segment (start 190 92.27) (end 189.187501 92.27) (width 0.6) (layer "F.Cu") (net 6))
 (segment (start 192 91.082499) (end 190.812499 92.27) (width 0.6) (layer "F.Cu") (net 6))
 (segment (start 192 90) (end 192 91.082499) (width 0.6) (layer "F.Cu") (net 6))
 (segment (start 190 88) (end 192 90) (width 0.6) (layer "F.Cu") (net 6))
 (segment (start 189.187501 92.27) (end 187.099001 94.3585) (width 0.6) (layer "F.Cu") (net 6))
 (segment (start 187.099001 94.3585) (end 187.099001 95.286453) (width 0.6) (layer "F.Cu") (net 6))
 (segment (start 190.812499 92.27) (end 190 92.27) (width 0.6) (layer "F.Cu") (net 6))
 (segment (start 189.812548 98) (end 191.08 98) (width 0.6) (layer "F.Cu") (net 6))
 (segment (start 191.08 98) (end 193.08 100) (width 0.6) (layer "F.Cu") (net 6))
 (segment (start 189.183295 91) (end 190 91) (width 0.6) (layer "F.Cu") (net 5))
 (segment (start 186.198002 93.985293) (end 189.183295 91) (width 0.6) (layer "F.Cu") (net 5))
 (segment (start 190.54 100) (end 186.198002 95.658002) (width 0.6) (layer "F.Cu") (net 5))
 (segment (start 186.198002 95.658002) (end 186.198002 93.985293) (width 0.6) (layer "F.Cu") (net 5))
 (segment (start 195 82) (end 193 80) (width 0.6) (layer "F.Cu") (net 2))
 (segment (start 195.7615 97.6015) (end 198.16 100) (width 0.6) (layer "F.Cu") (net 2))
 (segment (start 196.362501 93.54) (end 197.175 93.54) (width 0.6) (layer "F.Cu") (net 2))
 (segment (start 193 80) (end 193 79) (width 0.6) (layer "F.Cu") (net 2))
 (segment (start 196.548246 93.54) (end 195.7615 94.326746) (width 0.6) (layer "F.Cu") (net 2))
 (segment (start 197.175 93.54) (end 196.548246 93.54) (width 0.6) (layer "F.Cu") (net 2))
 (segment (start 194.8605 92.037999) (end 194.8605 82.1395) (width 0.6) (layer "F.Cu") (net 2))
 (segment (start 195.7615 94.326746) (end 195.7615 97.6015) (width 0.6) (layer "F.Cu") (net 2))
 (segment (start 196.362501 93.54) (end 194.8605 92.037999) (width 0.6) (layer "F.Cu") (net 2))
 (segment (start 194.8605 82.1395) (end 195 82) (width 0.6) (layer "F.Cu") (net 2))
 (segment (start 188 94.913246) (end 190.185754 97.099) (width 0.6) (layer "F.Cu") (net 7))
 (segment (start 192.719 97.099) (end 195.62 100) (width 0.6) (layer "F.Cu") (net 7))
 (segment (start 190 93.54) (end 189.373246 93.54) (width 0.6) (layer "F.Cu") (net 7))
 (segment (start 190.185754 97.099) (end 192.719 97.099) (width 0.6) (layer "F.Cu") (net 7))
 (segment (start 189.373246 93.54) (end 188 94.913246) (width 0.6) (layer "F.Cu") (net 7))
 (segment (start 198.05 94.81) (end 203.24 100) (width 0.6) (layer "F.Cu") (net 1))
 (segment (start 197.175 94.81) (end 198.05 94.81) (width 0.6) (layer "F.Cu") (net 1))
 (segment (start 195.7615 91.664793) (end 196.366707 92.27) (width 0.6) (layer "F.Cu") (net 3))
 (segment (start 197.175 92.27) (end 200.102024 92.27) (width 0.6) (layer "F.Cu") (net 3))
 (segment (start 207.231 99.398976) (end 207.231 100.601024) (width 0.6) (layer "F.Cu") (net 3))
 (segment (start 206.381024 101.451) (end 202.151 101.451) (width 0.6) (layer "F.Cu") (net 3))
 (segment (start 200.102024 92.27) (end 207.231 99.398976) (width 0.6) (layer "F.Cu") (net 3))
 (segment (start 195.7615 84.2385) (end 195.7615 91.664793) (width 0.6) (layer "F.Cu") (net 3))
 (segment (start 202.151 101.451) (end 200.7 100) (width 0.6) (layer "F.Cu") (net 3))
 (segment (start 201 79) (end 195.7615 84.2385) (width 0.6) (layer "F.Cu") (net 3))
 (segment (start 207.231 100.601024) (end 206.381024 101.451) (width 0.6) (layer "F.Cu") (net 3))
 (segment (start 196.366707 92.27) (end 197.175 92.27) (width 0.6) (layer "F.Cu") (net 3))
 (segment (start 178 88) (end 183 88) (width 0.6) (layer "F.Cu") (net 9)))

